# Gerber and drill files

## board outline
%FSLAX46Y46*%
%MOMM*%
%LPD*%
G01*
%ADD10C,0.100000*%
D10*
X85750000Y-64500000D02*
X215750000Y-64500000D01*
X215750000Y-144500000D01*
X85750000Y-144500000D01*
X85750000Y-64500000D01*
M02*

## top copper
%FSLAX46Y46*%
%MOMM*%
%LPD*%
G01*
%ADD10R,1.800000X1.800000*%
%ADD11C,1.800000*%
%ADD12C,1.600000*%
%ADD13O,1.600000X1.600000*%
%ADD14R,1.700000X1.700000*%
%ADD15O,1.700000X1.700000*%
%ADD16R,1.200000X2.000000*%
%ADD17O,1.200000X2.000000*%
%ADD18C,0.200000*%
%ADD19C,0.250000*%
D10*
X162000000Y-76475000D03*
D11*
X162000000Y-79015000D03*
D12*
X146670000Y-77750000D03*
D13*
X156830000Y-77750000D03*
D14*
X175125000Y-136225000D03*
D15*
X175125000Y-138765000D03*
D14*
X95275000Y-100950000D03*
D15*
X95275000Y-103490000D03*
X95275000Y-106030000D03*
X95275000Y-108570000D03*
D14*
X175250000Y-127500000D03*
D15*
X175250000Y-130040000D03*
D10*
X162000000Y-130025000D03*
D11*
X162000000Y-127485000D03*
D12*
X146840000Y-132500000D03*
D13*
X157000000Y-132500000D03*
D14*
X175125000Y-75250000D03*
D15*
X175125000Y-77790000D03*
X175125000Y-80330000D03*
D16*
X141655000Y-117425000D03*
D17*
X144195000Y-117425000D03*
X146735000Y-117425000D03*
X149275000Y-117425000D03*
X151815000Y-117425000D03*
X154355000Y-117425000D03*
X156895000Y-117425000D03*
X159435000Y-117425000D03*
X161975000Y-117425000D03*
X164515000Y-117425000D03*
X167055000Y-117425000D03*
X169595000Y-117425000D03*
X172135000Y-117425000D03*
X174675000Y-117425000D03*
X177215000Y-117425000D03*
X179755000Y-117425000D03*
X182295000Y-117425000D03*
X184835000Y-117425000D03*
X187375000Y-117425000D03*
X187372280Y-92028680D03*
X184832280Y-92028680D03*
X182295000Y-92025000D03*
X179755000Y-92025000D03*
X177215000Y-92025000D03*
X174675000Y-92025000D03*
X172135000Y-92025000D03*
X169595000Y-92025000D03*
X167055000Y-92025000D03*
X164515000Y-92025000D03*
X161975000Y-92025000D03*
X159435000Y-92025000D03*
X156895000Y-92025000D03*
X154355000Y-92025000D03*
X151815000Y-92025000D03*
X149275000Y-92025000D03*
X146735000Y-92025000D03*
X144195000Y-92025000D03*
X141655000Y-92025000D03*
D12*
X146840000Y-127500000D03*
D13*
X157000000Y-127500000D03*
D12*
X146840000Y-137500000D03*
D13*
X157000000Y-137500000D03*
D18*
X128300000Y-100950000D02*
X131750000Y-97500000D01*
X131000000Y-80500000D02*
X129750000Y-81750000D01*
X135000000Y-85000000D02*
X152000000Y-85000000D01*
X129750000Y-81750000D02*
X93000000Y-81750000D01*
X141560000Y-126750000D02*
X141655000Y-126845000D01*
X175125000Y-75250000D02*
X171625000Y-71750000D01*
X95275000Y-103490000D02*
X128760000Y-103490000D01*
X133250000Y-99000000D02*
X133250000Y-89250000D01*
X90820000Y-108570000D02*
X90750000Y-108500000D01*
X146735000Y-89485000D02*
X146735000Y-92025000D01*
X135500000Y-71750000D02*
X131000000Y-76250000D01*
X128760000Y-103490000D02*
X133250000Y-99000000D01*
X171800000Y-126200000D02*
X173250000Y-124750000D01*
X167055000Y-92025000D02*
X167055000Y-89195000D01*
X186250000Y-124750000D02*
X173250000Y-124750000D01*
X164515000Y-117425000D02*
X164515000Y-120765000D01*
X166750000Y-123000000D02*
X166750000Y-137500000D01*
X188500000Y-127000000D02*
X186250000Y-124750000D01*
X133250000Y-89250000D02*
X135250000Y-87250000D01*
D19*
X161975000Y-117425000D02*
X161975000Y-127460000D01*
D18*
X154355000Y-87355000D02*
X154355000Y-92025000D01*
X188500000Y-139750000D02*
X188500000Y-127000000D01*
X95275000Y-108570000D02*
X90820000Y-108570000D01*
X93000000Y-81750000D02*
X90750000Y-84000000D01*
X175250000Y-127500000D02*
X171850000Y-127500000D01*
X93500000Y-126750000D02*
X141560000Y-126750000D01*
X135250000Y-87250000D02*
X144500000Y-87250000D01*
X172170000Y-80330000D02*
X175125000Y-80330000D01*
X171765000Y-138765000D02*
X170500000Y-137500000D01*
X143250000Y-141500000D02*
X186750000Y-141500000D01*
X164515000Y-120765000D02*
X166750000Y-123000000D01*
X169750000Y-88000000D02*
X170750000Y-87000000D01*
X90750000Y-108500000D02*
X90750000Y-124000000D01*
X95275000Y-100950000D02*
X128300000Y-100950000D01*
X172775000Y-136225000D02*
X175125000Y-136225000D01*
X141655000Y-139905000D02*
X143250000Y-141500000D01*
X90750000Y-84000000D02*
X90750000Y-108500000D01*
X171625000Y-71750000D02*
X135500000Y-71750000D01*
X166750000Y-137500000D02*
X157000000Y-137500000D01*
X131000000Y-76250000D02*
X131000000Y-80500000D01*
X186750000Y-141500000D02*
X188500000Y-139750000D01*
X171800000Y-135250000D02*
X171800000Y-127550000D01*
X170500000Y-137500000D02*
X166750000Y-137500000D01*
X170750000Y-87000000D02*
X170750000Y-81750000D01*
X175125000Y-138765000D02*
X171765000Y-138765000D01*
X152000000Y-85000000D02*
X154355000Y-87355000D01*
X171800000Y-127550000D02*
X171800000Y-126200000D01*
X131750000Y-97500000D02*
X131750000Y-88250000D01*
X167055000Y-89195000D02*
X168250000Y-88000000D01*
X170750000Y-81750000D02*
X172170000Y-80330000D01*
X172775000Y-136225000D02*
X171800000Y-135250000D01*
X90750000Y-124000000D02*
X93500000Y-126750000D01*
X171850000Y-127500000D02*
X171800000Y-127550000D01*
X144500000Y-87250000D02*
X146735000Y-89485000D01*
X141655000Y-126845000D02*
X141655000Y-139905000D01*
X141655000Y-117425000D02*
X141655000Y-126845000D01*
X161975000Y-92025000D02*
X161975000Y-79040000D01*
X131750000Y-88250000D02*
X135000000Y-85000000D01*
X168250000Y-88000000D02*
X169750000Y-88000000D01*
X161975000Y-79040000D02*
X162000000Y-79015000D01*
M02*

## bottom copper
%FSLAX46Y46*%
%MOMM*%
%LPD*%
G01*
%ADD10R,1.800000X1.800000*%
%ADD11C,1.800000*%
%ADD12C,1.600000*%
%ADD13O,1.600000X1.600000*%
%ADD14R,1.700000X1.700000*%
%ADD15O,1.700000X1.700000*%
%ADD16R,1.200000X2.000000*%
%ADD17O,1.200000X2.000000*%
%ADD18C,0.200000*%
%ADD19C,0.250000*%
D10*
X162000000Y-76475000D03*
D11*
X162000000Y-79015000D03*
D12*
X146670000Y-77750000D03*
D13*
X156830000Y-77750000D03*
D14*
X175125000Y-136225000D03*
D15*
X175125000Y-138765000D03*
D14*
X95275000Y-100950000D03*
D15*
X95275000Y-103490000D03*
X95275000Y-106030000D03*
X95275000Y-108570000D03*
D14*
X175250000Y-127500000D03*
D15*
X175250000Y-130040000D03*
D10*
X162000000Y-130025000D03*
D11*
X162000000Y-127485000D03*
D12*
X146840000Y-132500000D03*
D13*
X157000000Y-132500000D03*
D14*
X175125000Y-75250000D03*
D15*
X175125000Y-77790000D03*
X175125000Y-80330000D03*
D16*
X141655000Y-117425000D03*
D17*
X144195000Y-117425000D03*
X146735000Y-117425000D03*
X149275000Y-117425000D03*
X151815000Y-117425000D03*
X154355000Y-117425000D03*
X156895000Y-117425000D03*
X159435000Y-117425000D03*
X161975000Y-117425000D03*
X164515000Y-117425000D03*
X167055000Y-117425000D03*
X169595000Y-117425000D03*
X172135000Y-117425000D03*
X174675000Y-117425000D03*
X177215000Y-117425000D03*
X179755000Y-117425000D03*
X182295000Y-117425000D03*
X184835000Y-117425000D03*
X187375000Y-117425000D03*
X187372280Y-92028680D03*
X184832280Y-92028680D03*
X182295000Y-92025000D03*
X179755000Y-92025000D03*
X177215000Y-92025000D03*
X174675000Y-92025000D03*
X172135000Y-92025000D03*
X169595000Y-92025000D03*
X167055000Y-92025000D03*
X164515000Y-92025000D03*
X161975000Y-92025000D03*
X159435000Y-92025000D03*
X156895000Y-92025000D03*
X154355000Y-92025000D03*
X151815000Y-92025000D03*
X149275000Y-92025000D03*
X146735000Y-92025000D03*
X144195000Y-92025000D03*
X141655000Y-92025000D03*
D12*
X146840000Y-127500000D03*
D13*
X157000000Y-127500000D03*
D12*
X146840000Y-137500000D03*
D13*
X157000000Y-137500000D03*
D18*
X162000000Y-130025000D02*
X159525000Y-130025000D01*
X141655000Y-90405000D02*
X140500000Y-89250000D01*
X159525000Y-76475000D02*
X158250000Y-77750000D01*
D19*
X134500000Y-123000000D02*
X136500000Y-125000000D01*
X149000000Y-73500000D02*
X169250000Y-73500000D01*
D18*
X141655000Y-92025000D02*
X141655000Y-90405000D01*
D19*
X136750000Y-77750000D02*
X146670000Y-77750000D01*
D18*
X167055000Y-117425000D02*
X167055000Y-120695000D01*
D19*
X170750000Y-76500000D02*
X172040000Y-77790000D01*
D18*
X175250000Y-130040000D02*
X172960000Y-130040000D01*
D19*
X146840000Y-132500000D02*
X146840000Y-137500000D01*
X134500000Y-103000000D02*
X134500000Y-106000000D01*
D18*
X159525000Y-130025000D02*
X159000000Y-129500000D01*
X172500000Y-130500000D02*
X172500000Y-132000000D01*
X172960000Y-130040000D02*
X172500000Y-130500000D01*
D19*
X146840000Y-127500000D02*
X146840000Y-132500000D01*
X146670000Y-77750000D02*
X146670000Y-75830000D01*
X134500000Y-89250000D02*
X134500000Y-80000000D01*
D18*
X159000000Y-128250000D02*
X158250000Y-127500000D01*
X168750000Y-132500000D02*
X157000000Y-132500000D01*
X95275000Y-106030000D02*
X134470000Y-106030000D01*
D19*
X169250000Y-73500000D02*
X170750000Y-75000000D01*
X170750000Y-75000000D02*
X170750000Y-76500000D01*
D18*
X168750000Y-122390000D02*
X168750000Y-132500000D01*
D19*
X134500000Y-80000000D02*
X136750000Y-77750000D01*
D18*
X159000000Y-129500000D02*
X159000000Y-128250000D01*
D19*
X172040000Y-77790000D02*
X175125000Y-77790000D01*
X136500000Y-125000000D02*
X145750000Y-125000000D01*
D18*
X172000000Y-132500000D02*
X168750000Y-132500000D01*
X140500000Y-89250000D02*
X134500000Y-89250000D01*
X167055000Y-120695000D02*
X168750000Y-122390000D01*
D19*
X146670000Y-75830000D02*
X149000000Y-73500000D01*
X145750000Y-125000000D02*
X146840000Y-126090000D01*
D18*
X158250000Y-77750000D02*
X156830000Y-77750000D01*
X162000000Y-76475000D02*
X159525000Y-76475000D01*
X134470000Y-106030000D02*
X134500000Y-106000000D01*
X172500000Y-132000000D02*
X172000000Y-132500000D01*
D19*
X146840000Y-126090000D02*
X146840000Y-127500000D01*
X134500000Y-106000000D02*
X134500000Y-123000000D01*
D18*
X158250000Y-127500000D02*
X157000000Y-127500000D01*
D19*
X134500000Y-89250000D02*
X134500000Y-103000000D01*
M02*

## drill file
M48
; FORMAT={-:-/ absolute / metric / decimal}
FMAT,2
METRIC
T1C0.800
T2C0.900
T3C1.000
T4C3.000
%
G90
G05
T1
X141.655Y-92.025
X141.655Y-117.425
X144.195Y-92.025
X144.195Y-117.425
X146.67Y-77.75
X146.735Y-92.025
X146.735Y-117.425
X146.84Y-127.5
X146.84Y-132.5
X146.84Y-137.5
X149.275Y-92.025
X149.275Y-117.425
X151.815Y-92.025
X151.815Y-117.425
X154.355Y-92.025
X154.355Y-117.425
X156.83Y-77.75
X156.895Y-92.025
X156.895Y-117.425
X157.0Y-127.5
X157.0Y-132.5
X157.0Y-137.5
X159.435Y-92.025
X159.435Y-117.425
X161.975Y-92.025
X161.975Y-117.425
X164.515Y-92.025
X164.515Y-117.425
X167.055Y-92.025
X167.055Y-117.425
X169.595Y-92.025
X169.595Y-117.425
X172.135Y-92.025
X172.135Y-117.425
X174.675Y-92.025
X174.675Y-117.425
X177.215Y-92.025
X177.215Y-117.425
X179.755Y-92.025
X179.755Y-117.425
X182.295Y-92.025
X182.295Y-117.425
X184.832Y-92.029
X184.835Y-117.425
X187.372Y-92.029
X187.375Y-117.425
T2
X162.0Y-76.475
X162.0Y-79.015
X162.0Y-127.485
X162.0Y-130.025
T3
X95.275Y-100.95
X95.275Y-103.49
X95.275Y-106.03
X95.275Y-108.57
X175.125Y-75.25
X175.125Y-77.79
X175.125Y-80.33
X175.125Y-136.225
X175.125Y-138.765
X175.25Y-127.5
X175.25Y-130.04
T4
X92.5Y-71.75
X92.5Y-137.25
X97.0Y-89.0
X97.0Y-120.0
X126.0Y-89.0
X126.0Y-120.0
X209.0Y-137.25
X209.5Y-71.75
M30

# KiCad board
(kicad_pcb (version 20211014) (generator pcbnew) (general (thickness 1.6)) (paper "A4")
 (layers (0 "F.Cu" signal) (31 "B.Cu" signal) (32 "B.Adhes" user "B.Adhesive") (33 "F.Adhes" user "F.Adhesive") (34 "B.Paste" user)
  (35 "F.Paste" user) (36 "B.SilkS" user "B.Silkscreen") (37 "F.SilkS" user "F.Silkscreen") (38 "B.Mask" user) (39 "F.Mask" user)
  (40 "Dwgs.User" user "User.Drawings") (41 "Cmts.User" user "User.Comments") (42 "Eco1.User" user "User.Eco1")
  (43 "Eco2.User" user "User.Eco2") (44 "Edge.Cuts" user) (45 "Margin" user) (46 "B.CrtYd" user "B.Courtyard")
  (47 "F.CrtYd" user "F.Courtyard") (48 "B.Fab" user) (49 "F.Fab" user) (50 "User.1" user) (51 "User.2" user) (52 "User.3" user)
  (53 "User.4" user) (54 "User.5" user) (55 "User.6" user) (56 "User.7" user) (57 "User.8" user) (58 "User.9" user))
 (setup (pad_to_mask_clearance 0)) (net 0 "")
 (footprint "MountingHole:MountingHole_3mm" (layer "F.Cu") (at 92.5 137.25)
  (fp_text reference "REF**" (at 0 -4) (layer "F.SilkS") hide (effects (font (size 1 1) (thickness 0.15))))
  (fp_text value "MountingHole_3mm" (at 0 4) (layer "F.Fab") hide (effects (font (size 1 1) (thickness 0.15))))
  (pad "" np_thru_hole circle (at 0 0) (size 3 3) (drill 3) (layers *.Cu *.Mask)))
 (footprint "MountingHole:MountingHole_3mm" (layer "F.Cu") (at 126 89)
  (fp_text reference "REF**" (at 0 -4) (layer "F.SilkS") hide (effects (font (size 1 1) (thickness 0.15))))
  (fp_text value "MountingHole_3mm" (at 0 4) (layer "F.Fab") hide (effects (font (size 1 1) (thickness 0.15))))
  (pad "" np_thru_hole circle (at 0 0) (size 3 3) (drill 3) (layers *.Cu *.Mask)))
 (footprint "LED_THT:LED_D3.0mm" (layer "F.Cu") (at 162 76.475 -90)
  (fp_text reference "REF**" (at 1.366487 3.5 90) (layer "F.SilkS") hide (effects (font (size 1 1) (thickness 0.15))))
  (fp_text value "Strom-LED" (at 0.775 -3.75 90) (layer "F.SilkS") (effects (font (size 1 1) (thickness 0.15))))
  (pad "1" thru_hole rect (at 0 0 270) (size 1.8 1.8) (drill 0.9) (layers *.Cu *.Mask))
  (pad "2" thru_hole circle (at 2.54 0 270) (size 1.8 1.8) (drill 0.9) (layers *.Cu *.Mask)))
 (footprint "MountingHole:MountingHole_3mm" (layer "F.Cu") (at 97 89)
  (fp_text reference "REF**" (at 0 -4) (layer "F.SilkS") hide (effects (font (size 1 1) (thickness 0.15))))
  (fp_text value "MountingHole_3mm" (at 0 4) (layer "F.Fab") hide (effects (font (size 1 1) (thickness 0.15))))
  (pad "" np_thru_hole circle (at 0 0) (size 3 3) (drill 3) (layers *.Cu *.Mask)))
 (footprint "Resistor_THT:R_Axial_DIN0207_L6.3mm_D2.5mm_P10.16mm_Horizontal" (layer "F.Cu") (at 146.67 77.75)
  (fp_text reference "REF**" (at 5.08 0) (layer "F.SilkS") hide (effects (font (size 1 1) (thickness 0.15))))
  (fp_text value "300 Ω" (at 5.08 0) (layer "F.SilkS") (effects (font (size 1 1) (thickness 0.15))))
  (pad "1" thru_hole circle (at 0 0) (size 1.6 1.6) (drill 0.8) (layers *.Cu *.Mask))
  (pad "2" thru_hole oval (at 10.16 0) (size 1.6 1.6) (drill 0.8) (layers *.Cu *.Mask)))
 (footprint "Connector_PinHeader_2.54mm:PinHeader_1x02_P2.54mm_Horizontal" (layer "F.Cu") (at 175.125 136.225)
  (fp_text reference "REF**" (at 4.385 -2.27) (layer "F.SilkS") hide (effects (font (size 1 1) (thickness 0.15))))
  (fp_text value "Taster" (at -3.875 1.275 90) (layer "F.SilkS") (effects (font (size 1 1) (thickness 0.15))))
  (pad "1" thru_hole rect (at 0 0) (size 1.7 1.7) (drill 1) (layers *.Cu *.Mask))
  (pad "2" thru_hole oval (at 0 2.54) (size 1.7 1.7) (drill 1) (layers *.Cu *.Mask)))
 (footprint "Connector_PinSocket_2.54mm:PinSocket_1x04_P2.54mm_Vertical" (layer "F.Cu") (at 95.275 100.95)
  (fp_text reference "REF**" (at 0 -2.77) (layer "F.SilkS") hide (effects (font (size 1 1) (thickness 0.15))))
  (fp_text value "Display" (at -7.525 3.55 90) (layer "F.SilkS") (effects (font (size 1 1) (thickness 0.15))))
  (pad "1" thru_hole rect (at 0 0) (size 1.7 1.7) (drill 1) (layers *.Cu *.Mask))
  (pad "2" thru_hole oval (at 0 2.54) (size 1.7 1.7) (drill 1) (layers *.Cu *.Mask))
  (pad "3" thru_hole oval (at 0 5.08) (size 1.7 1.7) (drill 1) (layers *.Cu *.Mask))
  (pad "4" thru_hole oval (at 0 7.62) (size 1.7 1.7) (drill 1) (layers *.Cu *.Mask)))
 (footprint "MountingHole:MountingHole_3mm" (layer "F.Cu") (at 126 120)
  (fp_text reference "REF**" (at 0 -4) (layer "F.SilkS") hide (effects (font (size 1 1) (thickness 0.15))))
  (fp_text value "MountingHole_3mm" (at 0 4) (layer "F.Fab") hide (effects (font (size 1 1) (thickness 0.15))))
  (pad "" np_thru_hole circle (at 0 0) (size 3 3) (drill 3) (layers *.Cu *.Mask)))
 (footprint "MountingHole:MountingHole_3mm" (layer "F.Cu") (at 92.5 71.75)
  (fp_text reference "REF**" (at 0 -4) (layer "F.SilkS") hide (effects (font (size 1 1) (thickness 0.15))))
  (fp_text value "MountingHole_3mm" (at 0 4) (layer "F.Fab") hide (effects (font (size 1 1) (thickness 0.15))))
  (pad "" np_thru_hole circle (at 0 0) (size 3 3) (drill 3) (layers *.Cu *.Mask)))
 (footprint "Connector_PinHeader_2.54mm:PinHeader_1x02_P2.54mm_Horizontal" (layer "F.Cu") (at 175.25 127.5)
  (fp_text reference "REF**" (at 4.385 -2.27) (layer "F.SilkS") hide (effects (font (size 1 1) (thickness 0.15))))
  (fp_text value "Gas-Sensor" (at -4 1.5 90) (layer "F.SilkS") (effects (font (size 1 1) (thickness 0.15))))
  (pad "1" thru_hole rect (at 0 0) (size 1.7 1.7) (drill 1) (layers *.Cu *.Mask))
  (pad "2" thru_hole oval (at 0 2.54) (size 1.7 1.7) (drill 1) (layers *.Cu *.Mask)))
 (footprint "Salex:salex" (layer "F.Cu") (at 117.25 74.75 90)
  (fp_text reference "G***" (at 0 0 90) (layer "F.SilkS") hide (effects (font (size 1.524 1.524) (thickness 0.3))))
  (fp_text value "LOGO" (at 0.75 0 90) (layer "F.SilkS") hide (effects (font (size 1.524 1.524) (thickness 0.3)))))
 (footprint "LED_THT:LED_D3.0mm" (layer "F.Cu") (at 162 130.025 90)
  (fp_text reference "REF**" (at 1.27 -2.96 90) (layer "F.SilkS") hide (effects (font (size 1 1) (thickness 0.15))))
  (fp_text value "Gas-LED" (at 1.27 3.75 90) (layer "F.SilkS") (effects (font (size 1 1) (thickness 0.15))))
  (pad "1" thru_hole rect (at 0 0 90) (size 1.8 1.8) (drill 0.9) (layers *.Cu *.Mask))
  (pad "2" thru_hole circle (at 2.54 0 90) (size 1.8 1.8) (drill 0.9) (layers *.Cu *.Mask)))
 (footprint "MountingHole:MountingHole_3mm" (layer "F.Cu") (at 209.5 71.75)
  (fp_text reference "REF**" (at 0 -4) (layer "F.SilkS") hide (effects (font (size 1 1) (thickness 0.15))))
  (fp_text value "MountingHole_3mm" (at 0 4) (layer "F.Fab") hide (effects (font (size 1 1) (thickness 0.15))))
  (pad "" np_thru_hole circle (at 0 0) (size 3 3) (drill 3) (layers *.Cu *.Mask)))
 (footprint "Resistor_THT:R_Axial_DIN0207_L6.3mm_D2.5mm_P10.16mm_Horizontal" (layer "F.Cu") (at 146.84 132.5)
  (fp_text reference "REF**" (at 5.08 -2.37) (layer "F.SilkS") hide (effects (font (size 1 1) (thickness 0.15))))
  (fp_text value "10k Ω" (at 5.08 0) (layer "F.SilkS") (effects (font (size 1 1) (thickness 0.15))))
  (pad "1" thru_hole circle (at 0 0) (size 1.6 1.6) (drill 0.8) (layers *.Cu *.Mask))
  (pad "2" thru_hole oval (at 10.16 0) (size 1.6 1.6) (drill 0.8) (layers *.Cu *.Mask)))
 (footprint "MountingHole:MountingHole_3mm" (layer "F.Cu") (at 209 137.25)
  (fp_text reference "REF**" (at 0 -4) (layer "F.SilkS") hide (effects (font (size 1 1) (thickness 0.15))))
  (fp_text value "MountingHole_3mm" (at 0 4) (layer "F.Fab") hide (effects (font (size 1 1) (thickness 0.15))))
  (pad "" np_thru_hole circle (at 0 0) (size 3 3) (drill 3) (layers *.Cu *.Mask)))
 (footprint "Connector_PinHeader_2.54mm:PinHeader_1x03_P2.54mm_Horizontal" (layer "F.Cu") (at 175.125 75.25)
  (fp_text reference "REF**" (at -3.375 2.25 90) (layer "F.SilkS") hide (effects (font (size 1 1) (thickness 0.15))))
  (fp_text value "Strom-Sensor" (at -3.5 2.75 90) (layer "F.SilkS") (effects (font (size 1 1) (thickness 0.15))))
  (pad "1" thru_hole rect (at 0 0) (size 1.7 1.7) (drill 1) (layers *.Cu *.Mask))
  (pad "2" thru_hole oval (at 0 2.54) (size 1.7 1.7) (drill 1) (layers *.Cu *.Mask))
  (pad "3" thru_hole oval (at 0 5.08) (size 1.7 1.7) (drill 1) (layers *.Cu *.Mask)))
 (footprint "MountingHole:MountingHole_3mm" (layer "F.Cu") (at 97 120)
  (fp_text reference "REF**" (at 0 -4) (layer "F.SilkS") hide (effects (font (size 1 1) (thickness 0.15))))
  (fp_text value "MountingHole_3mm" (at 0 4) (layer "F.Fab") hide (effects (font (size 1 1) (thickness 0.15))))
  (pad "" np_thru_hole circle (at 0 0) (size 3 3) (drill 3) (layers *.Cu *.Mask)))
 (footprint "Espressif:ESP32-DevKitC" (layer "F.Cu") (at 141.655 117.425 90)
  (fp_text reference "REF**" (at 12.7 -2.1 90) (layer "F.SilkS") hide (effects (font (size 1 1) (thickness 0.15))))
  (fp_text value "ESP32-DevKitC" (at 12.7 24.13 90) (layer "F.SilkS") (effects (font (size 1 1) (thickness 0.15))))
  (pad "1" thru_hole rect (at 0 0) (size 1.2 2) (drill 0.8) (layers *.Cu *.Mask))
  (pad "2" thru_hole oval (at 0 2.54) (size 1.2 2) (drill 0.8) (layers *.Cu *.Mask))
  (pad "3" thru_hole oval (at 0 5.08) (size 1.2 2) (drill 0.8) (layers *.Cu *.Mask))
  (pad "4" thru_hole oval (at 0 7.62) (size 1.2 2) (drill 0.8) (layers *.Cu *.Mask))
  (pad "5" thru_hole oval (at 0 10.16) (size 1.2 2) (drill 0.8) (layers *.Cu *.Mask))
  (pad "6" thru_hole oval (at 0 12.7) (size 1.2 2) (drill 0.8) (layers *.Cu *.Mask))
  (pad "7" thru_hole oval (at 0 15.24) (size 1.2 2) (drill 0.8) (layers *.Cu *.Mask))
  (pad "8" thru_hole oval (at 0 17.78) (size 1.2 2) (drill 0.8) (layers *.Cu *.Mask))
  (pad "9" thru_hole oval (at 0 20.32) (size 1.2 2) (drill 0.8) (layers *.Cu *.Mask))
  (pad "10" thru_hole oval (at 0 22.86) (size 1.2 2) (drill 0.8) (layers *.Cu *.Mask))
  (pad "11" thru_hole oval (at 0 25.4) (size 1.2 2) (drill 0.8) (layers *.Cu *.Mask))
  (pad "12" thru_hole oval (at 0 27.94) (size 1.2 2) (drill 0.8) (layers *.Cu *.Mask))
  (pad "13" thru_hole oval (at 0 30.48) (size 1.2 2) (drill 0.8) (layers *.Cu *.Mask))
  (pad "14" thru_hole oval (at 0 33.02) (size 1.2 2) (drill 0.8) (layers *.Cu *.Mask))
  (pad "15" thru_hole oval (at 0 35.56) (size 1.2 2) (drill 0.8) (layers *.Cu *.Mask))
  (pad "16" thru_hole oval (at 0 38.1) (size 1.2 2) (drill 0.8) (layers *.Cu *.Mask))
  (pad "17" thru_hole oval (at 0 40.64) (size 1.2 2) (drill 0.8) (layers *.Cu *.Mask))
  (pad "18" thru_hole oval (at 0 43.18) (size 1.2 2) (drill 0.8) (layers *.Cu *.Mask))
  (pad "19" thru_hole oval (at 0 45.72) (size 1.2 2) (drill 0.8) (layers *.Cu *.Mask))
  (pad "20" thru_hole oval (at 25.39632 45.71728) (size 1.2 2) (drill 0.8) (layers *.Cu *.Mask))
  (pad "21" thru_hole oval (at 25.39632 43.17728) (size 1.2 2) (drill 0.8) (layers *.Cu *.Mask))
  (pad "22" thru_hole oval (at 25.4 40.64) (size 1.2 2) (drill 0.8) (layers *.Cu *.Mask))
  (pad "23" thru_hole oval (at 25.4 38.1) (size 1.2 2) (drill 0.8) (layers *.Cu *.Mask))
  (pad "24" thru_hole oval (at 25.4 35.56) (size 1.2 2) (drill 0.8) (layers *.Cu *.Mask))
  (pad "25" thru_hole oval (at 25.4 33.02) (size 1.2 2) (drill 0.8) (layers *.Cu *.Mask))
  (pad "26" thru_hole oval (at 25.4 30.48) (size 1.2 2) (drill 0.8) (layers *.Cu *.Mask))
  (pad "27" thru_hole oval (at 25.4 27.94) (size 1.2 2) (drill 0.8) (layers *.Cu *.Mask))
  (pad "28" thru_hole oval (at 25.4 25.4) (size 1.2 2) (drill 0.8) (layers *.Cu *.Mask))
  (pad "29" thru_hole oval (at 25.4 22.86) (size 1.2 2) (drill 0.8) (layers *.Cu *.Mask))
  (pad "30" thru_hole oval (at 25.4 20.32) (size 1.2 2) (drill 0.8) (layers *.Cu *.Mask))
  (pad "31" thru_hole oval (at 25.4 17.78) (size 1.2 2) (drill 0.8) (layers *.Cu *.Mask))
  (pad "32" thru_hole oval (at 25.4 15.24) (size 1.2 2) (drill 0.8) (layers *.Cu *.Mask))
  (pad "33" thru_hole oval (at 25.4 12.7) (size 1.2 2) (drill 0.8) (layers *.Cu *.Mask))
  (pad "34" thru_hole oval (at 25.4 10.16) (size 1.2 2) (drill 0.8) (layers *.Cu *.Mask))
  (pad "35" thru_hole oval (at 25.4 7.62) (size 1.2 2) (drill 0.8) (layers *.Cu *.Mask))
  (pad "36" thru_hole oval (at 25.4 5.08) (size 1.2 2) (drill 0.8) (layers *.Cu *.Mask))
  (pad "37" thru_hole oval (at 25.4 2.54) (size 1.2 2) (drill 0.8) (layers *.Cu *.Mask))
  (pad "38" thru_hole oval (at 25.4 0) (size 1.2 2) (drill 0.8) (layers *.Cu *.Mask)))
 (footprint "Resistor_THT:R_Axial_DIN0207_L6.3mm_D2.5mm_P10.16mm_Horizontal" (layer "F.Cu") (at 146.84 127.5)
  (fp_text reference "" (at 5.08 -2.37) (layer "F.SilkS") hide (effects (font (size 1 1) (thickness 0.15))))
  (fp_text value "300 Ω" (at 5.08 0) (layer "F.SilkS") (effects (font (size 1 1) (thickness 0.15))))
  (pad "1" thru_hole circle (at 0 0) (size 1.6 1.6) (drill 0.8) (layers *.Cu *.Mask))
  (pad "2" thru_hole oval (at 10.16 0) (size 1.6 1.6) (drill 0.8) (layers *.Cu *.Mask)))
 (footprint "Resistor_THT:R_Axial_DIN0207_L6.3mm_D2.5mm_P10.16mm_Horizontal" (layer "F.Cu") (at 146.84 137.5)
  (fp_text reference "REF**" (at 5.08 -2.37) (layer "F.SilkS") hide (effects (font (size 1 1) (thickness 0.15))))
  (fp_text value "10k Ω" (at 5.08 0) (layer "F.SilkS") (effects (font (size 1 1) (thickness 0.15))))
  (pad "1" thru_hole circle (at 0 0) (size 1.6 1.6) (drill 0.8) (layers *.Cu *.Mask))
  (pad "2" thru_hole oval (at 10.16 0) (size 1.6 1.6) (drill 0.8) (layers *.Cu *.Mask)))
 (gr_rect (start 85.75 64.5) (end 215.75 144.5) (layer "Edge.Cuts") (width 0.1) (fill none))
 (segment (start 128.3 100.95) (end 131.75 97.5) (width 0.2) (layer "F.Cu") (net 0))
 (segment (start 131 80.5) (end 129.75 81.75) (width 0.2) (layer "F.Cu") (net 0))
 (segment (start 135 85) (end 152 85) (width 0.2) (layer "F.Cu") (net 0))
 (segment (start 129.75 81.75) (end 93 81.75) (width 0.2) (layer "F.Cu") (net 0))
 (segment (start 141.56 126.75) (end 141.655 126.845) (width 0.2) (layer "F.Cu") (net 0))
 (segment (start 175.125 75.25) (end 171.625 71.75) (width 0.2) (layer "F.Cu") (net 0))
 (segment (start 95.275 103.49) (end 128.76 103.49) (width 0.2) (layer "F.Cu") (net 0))
 (segment (start 133.25 99) (end 133.25 89.25) (width 0.2) (layer "F.Cu") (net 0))
 (segment (start 90.82 108.57) (end 90.75 108.5) (width 0.2) (layer "F.Cu") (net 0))
 (segment (start 146.735 89.485) (end 146.735 92.025) (width 0.2) (layer "F.Cu") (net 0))
 (segment (start 135.5 71.75) (end 131 76.25) (width 0.2) (layer "F.Cu") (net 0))
 (segment (start 128.76 103.49) (end 133.25 99) (width 0.2) (layer "F.Cu") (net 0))
 (segment (start 171.8 126.2) (end 173.25 124.75) (width 0.2) (layer "F.Cu") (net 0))
 (segment (start 167.055 92.025) (end 167.055 89.195) (width 0.2) (layer "F.Cu") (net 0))
 (segment (start 186.25 124.75) (end 173.25 124.75) (width 0.2) (layer "F.Cu") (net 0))
 (segment (start 164.515 117.425) (end 164.515 120.765) (width 0.2) (layer "F.Cu") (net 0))
 (segment (start 166.75 123) (end 166.75 137.5) (width 0.2) (layer "F.Cu") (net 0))
 (segment (start 188.5 127) (end 186.25 124.75) (width 0.2) (layer "F.Cu") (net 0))
 (segment (start 133.25 89.25) (end 135.25 87.25) (width 0.2) (layer "F.Cu") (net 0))
 (segment (start 161.975 117.425) (end 161.975 127.46) (width 0.25) (layer "F.Cu") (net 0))
 (segment (start 154.355 87.355) (end 154.355 92.025) (width 0.2) (layer "F.Cu") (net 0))
 (segment (start 188.5 139.75) (end 188.5 127) (width 0.2) (layer "F.Cu") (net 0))
 (segment (start 95.275 108.57) (end 90.82 108.57) (width 0.2) (layer "F.Cu") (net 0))
 (segment (start 93 81.75) (end 90.75 84) (width 0.2) (layer "F.Cu") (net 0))
 (segment (start 175.25 127.5) (end 171.85 127.5) (width 0.2) (layer "F.Cu") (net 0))
 (segment (start 93.5 126.75) (end 141.56 126.75) (width 0.2) (layer "F.Cu") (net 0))
 (segment (start 135.25 87.25) (end 144.5 87.25) (width 0.2) (layer "F.Cu") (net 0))
 (segment (start 172.17 80.33) (end 175.125 80.33) (width 0.2) (layer "F.Cu") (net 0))
 (segment (start 171.765 138.765) (end 170.5 137.5) (width 0.2) (layer "F.Cu") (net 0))
 (segment (start 143.25 141.5) (end 186.75 141.5) (width 0.2) (layer "F.Cu") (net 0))
 (segment (start 164.515 120.765) (end 166.75 123) (width 0.2) (layer "F.Cu") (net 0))
 (segment (start 169.75 88) (end 170.75 87) (width 0.2) (layer "F.Cu") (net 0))
 (segment (start 90.75 108.5) (end 90.75 124) (width 0.2) (layer "F.Cu") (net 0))
 (segment (start 95.275 100.95) (end 128.3 100.95) (width 0.2) (layer "F.Cu") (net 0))
 (segment (start 172.775 136.225) (end 175.125 136.225) (width 0.2) (layer "F.Cu") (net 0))
 (segment (start 141.655 139.905) (end 143.25 141.5) (width 0.2) (layer "F.Cu") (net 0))
 (segment (start 90.75 84) (end 90.75 108.5) (width 0.2) (layer "F.Cu") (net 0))
 (segment (start 171.625 71.75) (end 135.5 71.75) (width 0.2) (layer "F.Cu") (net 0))
 (segment (start 166.75 137.5) (end 157 137.5) (width 0.2) (layer "F.Cu") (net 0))
 (segment (start 131 76.25) (end 131 80.5) (width 0.2) (layer "F.Cu") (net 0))
 (segment (start 186.75 141.5) (end 188.5 139.75) (width 0.2) (layer "F.Cu") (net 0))
 (segment (start 171.8 135.25) (end 171.8 127.55) (width 0.2) (layer "F.Cu") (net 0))
 (segment (start 170.5 137.5) (end 166.75 137.5) (width 0.2) (layer "F.Cu") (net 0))
 (segment (start 170.75 87) (end 170.75 81.75) (width 0.2) (layer "F.Cu") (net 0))
 (segment (start 175.125 138.765) (end 171.765 138.765) (width 0.2) (layer "F.Cu") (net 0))
 (segment (start 152 85) (end 154.355 87.355) (width 0.2) (layer "F.Cu") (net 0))
 (segment (start 171.8 127.55) (end 171.8 126.2) (width 0.2) (layer "F.Cu") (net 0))
 (segment (start 131.75 97.5) (end 131.75 88.25) (width 0.2) (layer "F.Cu") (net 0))
 (segment (start 167.055 89.195) (end 168.25 88) (width 0.2) (layer "F.Cu") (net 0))
 (segment (start 170.75 81.75) (end 172.17 80.33) (width 0.2) (layer "F.Cu") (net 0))
 (segment (start 172.775 136.225) (end 171.8 135.25) (width 0.2) (layer "F.Cu") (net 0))
 (segment (start 90.75 124) (end 93.5 126.75) (width 0.2) (layer "F.Cu") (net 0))
 (segment (start 171.85 127.5) (end 171.8 127.55) (width 0.2) (layer "F.Cu") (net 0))
 (segment (start 144.5 87.25) (end 146.735 89.485) (width 0.2) (layer "F.Cu") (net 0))
 (segment (start 141.655 126.845) (end 141.655 139.905) (width 0.2) (layer "F.Cu") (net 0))
 (segment (start 141.655 117.425) (end 141.655 126.845) (width 0.2) (layer "F.Cu") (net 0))
 (segment (start 161.975 92.025) (end 161.975 79.04) (width 0.2) (layer "F.Cu") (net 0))
 (segment (start 131.75 88.25) (end 135 85) (width 0.2) (layer "F.Cu") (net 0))
 (segment (start 168.25 88) (end 169.75 88) (width 0.2) (layer "F.Cu") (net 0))
 (segment (start 161.975 79.04) (end 162 79.015) (width 0.2) (layer "F.Cu") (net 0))
 (segment (start 162 130.025) (end 159.525 130.025) (width 0.2) (layer "B.Cu") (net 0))
 (segment (start 141.655 90.405) (end 140.5 89.25) (width 0.2) (layer "B.Cu") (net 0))
 (segment (start 159.525 76.475) (end 158.25 77.75) (width 0.2) (layer "B.Cu") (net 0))
 (segment (start 134.5 123) (end 136.5 125) (width 0.25) (layer "B.Cu") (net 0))
 (segment (start 149 73.5) (end 169.25 73.5) (width 0.25) (layer "B.Cu") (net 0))
 (segment (start 141.655 92.025) (end 141.655 90.405) (width 0.2) (layer "B.Cu") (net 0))
 (segment (start 136.75 77.75) (end 146.67 77.75) (width 0.25) (layer "B.Cu") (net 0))
 (segment (start 167.055 117.425) (end 167.055 120.695) (width 0.2) (layer "B.Cu") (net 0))
 (segment (start 170.75 76.5) (end 172.04 77.79) (width 0.25) (layer "B.Cu") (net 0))
 (segment (start 175.25 130.04) (end 172.96 130.04) (width 0.2) (layer "B.Cu") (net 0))
 (segment (start 146.84 132.5) (end 146.84 137.5) (width 0.25) (layer "B.Cu") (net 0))
 (segment (start 134.5 103) (end 134.5 106) (width 0.25) (layer "B.Cu") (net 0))
 (segment (start 159.525 130.025) (end 159 129.5) (width 0.2) (layer "B.Cu") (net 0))
 (segment (start 172.5 130.5) (end 172.5 132) (width 0.2) (layer "B.Cu") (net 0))
 (segment (start 172.96 130.04) (end 172.5 130.5) (width 0.2) (layer "B.Cu") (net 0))
 (segment (start 146.84 127.5) (end 146.84 132.5) (width 0.25) (layer "B.Cu") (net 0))
 (segment (start 146.67 77.75) (end 146.67 75.83) (width 0.25) (layer "B.Cu") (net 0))
 (segment (start 134.5 89.25) (end 134.5 80) (width 0.25) (layer "B.Cu") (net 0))
 (segment (start 159 128.25) (end 158.25 127.5) (width 0.2) (layer "B.Cu") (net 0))
 (segment (start 168.75 132.5) (end 157 132.5) (width 0.2) (layer "B.Cu") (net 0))
 (segment (start 95.275 106.03) (end 134.47 106.03) (width 0.2) (layer "B.Cu") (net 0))
 (segment (start 169.25 73.5) (end 170.75 75) (width 0.25) (layer "B.Cu") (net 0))
 (segment (start 170.75 75) (end 170.75 76.5) (width 0.25) (layer "B.Cu") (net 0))
 (segment (start 168.75 122.39) (end 168.75 132.5) (width 0.2) (layer "B.Cu") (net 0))
 (segment (start 134.5 80) (end 136.75 77.75) (width 0.25) (layer "B.Cu") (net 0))
 (segment (start 159 129.5) (end 159 128.25) (width 0.2) (layer "B.Cu") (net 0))
 (segment (start 172.04 77.79) (end 175.125 77.79) (width 0.25) (layer "B.Cu") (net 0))
 (segment (start 136.5 125) (end 145.75 125) (width 0.25) (layer "B.Cu") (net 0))
 (segment (start 172 132.5) (end 168.75 132.5) (width 0.2) (layer "B.Cu") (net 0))
 (segment (start 140.5 89.25) (end 134.5 89.25) (width 0.2) (layer "B.Cu") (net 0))
 (segment (start 167.055 120.695) (end 168.75 122.39) (width 0.2) (layer "B.Cu") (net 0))
 (segment (start 146.67 75.83) (end 149 73.5) (width 0.25) (layer "B.Cu") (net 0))
 (segment (start 145.75 125) (end 146.84 126.09) (width 0.25) (layer "B.Cu") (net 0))
 (segment (start 158.25 77.75) (end 156.83 77.75) (width 0.2) (layer "B.Cu") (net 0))
 (segment (start 162 76.475) (end 159.525 76.475) (width 0.2) (layer "B.Cu") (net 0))
 (segment (start 134.47 106.03) (end 134.5 106) (width 0.2) (layer "B.Cu") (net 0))
 (segment (start 172.5 132) (end 172 132.5) (width 0.2) (layer "B.Cu") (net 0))
 (segment (start 146.84 126.09) (end 146.84 127.5) (width 0.25) (layer "B.Cu") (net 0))
 (segment (start 134.5 106) (end 134.5 123) (width 0.25) (layer "B.Cu") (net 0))
 (segment (start 158.25 127.5) (end 157 127.5) (width 0.2) (layer "B.Cu") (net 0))
 (segment (start 134.5 89.25) (end 134.5 103) (width 0.25) (layer "B.Cu") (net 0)))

